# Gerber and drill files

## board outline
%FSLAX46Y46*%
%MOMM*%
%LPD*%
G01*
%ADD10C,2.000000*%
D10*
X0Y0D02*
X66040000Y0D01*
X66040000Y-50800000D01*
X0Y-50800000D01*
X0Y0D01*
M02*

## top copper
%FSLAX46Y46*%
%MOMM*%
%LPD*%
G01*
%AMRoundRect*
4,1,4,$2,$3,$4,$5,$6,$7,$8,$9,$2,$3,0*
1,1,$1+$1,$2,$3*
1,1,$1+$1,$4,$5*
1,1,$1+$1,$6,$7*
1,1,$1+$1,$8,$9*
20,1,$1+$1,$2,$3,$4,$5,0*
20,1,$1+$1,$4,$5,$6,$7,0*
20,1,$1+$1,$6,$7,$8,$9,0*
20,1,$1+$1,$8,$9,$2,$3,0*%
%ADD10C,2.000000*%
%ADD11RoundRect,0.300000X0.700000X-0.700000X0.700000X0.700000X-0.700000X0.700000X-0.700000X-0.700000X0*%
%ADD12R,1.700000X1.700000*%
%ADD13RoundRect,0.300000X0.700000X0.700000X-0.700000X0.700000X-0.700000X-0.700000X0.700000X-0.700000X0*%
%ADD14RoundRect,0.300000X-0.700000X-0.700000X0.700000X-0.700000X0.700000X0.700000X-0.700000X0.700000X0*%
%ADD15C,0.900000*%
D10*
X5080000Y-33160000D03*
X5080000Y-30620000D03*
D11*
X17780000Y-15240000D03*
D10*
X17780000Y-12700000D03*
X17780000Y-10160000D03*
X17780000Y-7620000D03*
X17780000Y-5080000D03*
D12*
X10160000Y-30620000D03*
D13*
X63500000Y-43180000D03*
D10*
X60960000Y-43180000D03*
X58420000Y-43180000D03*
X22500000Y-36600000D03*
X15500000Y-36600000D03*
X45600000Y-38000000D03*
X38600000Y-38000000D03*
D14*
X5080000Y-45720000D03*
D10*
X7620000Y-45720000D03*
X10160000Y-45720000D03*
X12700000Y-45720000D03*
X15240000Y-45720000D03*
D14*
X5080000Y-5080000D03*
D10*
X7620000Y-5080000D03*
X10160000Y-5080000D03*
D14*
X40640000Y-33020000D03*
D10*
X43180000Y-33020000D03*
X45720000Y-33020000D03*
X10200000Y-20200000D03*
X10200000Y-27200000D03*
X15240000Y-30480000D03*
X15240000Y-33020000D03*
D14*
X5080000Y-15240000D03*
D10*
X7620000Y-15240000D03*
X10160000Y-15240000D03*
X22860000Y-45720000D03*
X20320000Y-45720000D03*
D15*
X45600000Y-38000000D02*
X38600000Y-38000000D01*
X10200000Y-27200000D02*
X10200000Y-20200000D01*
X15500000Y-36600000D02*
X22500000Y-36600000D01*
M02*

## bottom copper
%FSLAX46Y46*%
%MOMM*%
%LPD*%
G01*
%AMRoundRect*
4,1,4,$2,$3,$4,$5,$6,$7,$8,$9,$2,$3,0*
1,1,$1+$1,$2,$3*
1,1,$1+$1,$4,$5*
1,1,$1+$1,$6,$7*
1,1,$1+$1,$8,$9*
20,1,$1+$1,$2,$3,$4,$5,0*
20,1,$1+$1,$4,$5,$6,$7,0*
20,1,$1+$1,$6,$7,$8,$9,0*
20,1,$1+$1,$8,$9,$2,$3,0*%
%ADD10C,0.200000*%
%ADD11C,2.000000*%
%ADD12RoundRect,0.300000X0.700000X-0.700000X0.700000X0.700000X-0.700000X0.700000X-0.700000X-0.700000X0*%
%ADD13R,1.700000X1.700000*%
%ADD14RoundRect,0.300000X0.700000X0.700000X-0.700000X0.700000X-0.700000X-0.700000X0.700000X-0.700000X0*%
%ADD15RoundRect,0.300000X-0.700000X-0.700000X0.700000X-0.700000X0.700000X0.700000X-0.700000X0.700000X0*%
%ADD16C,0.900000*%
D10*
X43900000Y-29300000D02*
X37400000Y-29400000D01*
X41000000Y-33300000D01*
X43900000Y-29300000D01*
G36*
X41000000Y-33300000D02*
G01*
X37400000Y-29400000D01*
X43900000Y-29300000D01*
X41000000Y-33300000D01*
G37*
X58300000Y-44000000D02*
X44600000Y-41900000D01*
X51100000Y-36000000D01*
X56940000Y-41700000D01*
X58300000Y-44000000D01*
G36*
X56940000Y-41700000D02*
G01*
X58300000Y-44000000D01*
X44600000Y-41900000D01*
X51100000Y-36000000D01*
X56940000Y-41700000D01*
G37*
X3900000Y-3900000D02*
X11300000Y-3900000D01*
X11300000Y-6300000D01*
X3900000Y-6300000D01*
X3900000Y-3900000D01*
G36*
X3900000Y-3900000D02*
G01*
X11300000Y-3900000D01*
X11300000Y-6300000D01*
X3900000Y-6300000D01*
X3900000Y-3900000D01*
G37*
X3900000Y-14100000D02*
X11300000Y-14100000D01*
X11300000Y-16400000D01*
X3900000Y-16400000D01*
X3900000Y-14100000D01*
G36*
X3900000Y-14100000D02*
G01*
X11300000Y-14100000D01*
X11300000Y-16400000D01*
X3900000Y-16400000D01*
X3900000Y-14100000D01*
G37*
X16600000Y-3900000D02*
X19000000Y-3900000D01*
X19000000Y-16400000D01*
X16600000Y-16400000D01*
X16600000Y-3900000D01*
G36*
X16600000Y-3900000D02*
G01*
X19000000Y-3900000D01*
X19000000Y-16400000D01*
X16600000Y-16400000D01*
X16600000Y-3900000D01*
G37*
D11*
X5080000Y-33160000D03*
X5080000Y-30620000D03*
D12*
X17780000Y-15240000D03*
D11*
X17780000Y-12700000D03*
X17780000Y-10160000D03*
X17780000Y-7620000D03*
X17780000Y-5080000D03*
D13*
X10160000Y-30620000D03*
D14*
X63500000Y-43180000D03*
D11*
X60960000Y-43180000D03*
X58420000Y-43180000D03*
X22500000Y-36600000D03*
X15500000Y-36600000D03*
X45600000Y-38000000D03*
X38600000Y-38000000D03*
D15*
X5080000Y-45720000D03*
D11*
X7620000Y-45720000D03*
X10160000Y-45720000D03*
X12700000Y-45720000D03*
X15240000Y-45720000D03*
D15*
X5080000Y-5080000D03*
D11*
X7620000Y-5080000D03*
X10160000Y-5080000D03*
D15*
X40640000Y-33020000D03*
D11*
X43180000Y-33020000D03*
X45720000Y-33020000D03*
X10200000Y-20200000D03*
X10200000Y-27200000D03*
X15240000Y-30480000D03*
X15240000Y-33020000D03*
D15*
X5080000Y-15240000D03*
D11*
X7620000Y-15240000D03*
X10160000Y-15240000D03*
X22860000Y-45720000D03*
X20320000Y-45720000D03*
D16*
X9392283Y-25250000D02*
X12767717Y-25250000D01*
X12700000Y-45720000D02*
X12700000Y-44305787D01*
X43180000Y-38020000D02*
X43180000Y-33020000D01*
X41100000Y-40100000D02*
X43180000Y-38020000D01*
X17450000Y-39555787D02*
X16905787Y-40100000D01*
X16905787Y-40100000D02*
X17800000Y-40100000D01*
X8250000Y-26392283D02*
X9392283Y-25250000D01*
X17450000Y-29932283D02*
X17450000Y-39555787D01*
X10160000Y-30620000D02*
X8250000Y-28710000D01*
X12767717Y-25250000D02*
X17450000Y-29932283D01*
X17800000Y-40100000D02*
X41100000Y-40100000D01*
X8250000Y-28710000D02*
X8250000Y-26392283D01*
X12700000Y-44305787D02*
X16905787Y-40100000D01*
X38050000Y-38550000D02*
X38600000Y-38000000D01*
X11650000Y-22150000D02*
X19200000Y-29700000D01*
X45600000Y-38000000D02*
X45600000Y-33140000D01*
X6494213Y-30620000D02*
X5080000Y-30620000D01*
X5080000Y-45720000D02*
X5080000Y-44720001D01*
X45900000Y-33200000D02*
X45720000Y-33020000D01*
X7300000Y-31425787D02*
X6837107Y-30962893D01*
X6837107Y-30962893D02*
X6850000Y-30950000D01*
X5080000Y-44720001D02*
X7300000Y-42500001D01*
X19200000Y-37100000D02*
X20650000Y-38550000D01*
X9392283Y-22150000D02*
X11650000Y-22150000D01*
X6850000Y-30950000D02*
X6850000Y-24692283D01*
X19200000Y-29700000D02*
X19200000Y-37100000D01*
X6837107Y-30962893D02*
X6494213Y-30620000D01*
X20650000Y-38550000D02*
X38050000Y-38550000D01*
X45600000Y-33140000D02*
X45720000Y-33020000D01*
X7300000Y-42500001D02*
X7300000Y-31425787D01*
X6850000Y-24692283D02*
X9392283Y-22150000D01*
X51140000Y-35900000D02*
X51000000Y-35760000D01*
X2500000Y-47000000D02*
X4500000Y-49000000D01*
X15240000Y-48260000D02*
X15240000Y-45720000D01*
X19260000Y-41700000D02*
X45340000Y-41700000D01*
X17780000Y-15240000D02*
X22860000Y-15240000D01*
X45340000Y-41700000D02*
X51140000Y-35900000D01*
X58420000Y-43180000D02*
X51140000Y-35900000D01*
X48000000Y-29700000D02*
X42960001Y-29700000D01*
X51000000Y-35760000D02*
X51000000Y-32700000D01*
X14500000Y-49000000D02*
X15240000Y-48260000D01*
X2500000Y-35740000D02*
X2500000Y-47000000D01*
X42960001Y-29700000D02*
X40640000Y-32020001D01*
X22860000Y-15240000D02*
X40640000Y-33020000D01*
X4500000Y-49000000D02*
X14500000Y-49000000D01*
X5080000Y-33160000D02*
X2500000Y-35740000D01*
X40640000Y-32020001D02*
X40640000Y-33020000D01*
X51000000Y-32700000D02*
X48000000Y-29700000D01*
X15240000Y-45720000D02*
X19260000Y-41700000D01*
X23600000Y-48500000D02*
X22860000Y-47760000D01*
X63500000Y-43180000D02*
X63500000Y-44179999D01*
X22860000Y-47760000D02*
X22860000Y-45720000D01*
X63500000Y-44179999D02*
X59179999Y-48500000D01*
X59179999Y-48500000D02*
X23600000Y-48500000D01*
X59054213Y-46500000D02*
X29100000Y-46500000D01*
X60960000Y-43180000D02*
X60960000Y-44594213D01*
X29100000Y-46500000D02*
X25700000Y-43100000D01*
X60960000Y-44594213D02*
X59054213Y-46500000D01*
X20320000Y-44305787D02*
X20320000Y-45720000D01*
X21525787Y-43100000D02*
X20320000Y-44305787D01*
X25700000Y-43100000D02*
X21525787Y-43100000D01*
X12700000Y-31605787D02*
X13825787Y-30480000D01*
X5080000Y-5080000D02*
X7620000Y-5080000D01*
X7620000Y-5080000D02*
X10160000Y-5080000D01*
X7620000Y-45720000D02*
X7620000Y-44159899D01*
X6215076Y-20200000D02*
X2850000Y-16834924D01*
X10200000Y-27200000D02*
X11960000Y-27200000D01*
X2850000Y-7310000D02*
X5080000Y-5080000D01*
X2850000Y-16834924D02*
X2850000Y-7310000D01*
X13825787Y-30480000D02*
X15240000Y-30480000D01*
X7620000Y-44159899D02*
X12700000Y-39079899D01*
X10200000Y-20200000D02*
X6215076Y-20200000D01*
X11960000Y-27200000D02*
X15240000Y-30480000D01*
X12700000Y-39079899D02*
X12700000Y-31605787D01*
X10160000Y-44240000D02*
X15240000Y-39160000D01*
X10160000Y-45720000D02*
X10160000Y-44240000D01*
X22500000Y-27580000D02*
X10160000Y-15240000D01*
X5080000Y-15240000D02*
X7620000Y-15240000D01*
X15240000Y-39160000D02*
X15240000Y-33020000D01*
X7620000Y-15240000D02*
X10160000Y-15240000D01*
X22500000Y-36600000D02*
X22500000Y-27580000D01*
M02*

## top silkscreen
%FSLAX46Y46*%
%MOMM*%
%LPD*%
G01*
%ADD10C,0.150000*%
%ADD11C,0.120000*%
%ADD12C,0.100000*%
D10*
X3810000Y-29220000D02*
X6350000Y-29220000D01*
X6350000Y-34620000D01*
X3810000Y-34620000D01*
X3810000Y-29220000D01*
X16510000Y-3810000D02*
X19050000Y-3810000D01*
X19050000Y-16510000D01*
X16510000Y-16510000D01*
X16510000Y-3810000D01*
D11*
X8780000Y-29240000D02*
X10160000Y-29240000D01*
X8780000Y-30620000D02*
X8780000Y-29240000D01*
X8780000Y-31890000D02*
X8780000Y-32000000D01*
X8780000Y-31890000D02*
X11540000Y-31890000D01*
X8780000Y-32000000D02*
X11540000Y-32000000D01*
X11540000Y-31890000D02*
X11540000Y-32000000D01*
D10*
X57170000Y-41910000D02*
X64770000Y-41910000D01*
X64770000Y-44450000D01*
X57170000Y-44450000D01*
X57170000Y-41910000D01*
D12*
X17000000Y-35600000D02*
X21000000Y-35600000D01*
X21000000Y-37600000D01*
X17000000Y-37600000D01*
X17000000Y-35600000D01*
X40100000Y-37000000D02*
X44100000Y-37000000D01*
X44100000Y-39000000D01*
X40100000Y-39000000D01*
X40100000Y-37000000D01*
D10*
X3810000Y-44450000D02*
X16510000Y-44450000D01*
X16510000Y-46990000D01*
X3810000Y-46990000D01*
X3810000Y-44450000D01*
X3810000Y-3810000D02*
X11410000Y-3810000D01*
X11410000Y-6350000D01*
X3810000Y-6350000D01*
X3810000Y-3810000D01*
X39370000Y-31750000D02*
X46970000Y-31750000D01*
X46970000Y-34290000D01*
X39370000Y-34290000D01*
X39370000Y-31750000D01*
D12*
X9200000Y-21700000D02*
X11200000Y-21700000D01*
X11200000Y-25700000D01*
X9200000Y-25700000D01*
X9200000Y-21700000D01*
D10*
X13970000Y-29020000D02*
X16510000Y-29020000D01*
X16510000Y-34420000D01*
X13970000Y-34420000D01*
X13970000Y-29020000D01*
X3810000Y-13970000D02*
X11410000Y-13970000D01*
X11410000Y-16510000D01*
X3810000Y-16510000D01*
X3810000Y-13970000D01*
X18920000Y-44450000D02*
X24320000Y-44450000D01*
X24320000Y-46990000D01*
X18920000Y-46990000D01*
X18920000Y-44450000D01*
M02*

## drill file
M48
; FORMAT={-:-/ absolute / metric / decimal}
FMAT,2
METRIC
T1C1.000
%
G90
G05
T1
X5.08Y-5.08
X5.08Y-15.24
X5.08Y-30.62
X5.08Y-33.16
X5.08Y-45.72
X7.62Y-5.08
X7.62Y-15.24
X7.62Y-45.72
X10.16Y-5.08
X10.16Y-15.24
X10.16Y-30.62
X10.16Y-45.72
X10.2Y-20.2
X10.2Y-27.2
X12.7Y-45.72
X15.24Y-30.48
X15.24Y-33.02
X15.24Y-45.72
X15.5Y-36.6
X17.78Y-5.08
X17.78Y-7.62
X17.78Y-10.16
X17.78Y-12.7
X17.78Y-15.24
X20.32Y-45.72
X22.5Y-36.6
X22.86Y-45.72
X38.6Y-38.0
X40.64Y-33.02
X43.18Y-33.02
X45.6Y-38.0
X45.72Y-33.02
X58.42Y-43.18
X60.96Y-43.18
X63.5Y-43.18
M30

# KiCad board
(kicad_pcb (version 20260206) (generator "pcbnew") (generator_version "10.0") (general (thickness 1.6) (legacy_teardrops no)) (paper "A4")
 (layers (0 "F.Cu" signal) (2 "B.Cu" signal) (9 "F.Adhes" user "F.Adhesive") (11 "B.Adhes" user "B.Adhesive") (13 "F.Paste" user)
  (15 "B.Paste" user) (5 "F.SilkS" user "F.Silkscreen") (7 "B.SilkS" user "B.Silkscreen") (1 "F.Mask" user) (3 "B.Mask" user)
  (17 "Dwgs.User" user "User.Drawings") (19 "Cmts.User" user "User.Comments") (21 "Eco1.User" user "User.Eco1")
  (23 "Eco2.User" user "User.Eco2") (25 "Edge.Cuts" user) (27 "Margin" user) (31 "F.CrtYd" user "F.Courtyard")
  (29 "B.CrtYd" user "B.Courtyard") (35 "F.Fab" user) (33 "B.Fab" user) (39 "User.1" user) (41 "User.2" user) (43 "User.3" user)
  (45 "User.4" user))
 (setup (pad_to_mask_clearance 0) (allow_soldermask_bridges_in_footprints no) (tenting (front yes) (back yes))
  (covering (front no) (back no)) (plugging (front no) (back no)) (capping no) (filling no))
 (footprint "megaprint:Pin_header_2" (layer "F.Cu") (at 5.08 31.82 90)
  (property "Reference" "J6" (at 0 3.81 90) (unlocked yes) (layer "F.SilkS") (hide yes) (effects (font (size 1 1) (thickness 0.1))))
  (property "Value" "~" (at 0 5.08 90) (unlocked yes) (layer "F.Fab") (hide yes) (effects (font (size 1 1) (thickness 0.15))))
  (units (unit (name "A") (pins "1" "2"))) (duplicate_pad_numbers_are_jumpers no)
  (fp_rect (start -2.8 -1.27) (end 2.6 1.27) (stroke (width 0.15) (type default)) (fill no) (layer "F.SilkS"))
  (pad "1" thru_hole circle (at -1.34 0 90) (size 2 2) (drill 1) (layers "*.Cu" "*.Mask") (remove_unused_layers no) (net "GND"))
  (pad "2" thru_hole circle (at 1.2 0 90) (size 2 2) (drill 1) (layers "*.Cu" "*.Mask") (remove_unused_layers no) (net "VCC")))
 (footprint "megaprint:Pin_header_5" (layer "F.Cu") (at 17.78 10.16 90)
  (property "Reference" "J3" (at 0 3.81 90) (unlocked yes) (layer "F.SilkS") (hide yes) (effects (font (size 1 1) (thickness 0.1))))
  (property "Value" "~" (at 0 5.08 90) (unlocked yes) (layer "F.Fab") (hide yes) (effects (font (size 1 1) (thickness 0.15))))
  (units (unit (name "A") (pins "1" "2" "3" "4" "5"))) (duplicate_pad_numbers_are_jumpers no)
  (fp_rect (start -6.35 -1.27) (end 6.35 1.27) (stroke (width 0.15) (type default)) (fill no) (layer "F.SilkS"))
  (pad "1" thru_hole roundrect (at -5.08 0 90) (size 2 2) (drill 1) (layers "*.Cu" "*.Mask") (remove_unused_layers no)
   (roundrect_rratio 0.15) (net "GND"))
  (pad "2" thru_hole circle (at -2.54 0 90) (size 2 2) (drill 1) (layers "*.Cu" "*.Mask") (remove_unused_layers no) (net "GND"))
  (pad "3" thru_hole circle (at 0 0 90) (size 2 2) (drill 1) (layers "*.Cu" "*.Mask") (remove_unused_layers no) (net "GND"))
  (pad "4" thru_hole circle (at 2.54 0 90) (size 2 2) (drill 1) (layers "*.Cu" "*.Mask") (remove_unused_layers no) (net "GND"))
  (pad "5" thru_hole circle (at 5.08 0 90) (size 2 2) (drill 1) (layers "*.Cu" "*.Mask") (remove_unused_layers no) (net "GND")))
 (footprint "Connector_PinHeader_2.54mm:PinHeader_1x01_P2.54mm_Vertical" (layer "F.Cu") (at 10.16 30.62)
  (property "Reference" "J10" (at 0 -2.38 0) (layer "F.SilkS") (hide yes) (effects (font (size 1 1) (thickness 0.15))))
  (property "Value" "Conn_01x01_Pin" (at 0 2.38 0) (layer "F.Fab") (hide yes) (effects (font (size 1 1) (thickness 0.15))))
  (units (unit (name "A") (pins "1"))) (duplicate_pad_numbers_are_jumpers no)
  (fp_line (start -1.38 -1.38) (end 0 -1.38) (stroke (width 0.12) (type solid)) (layer "F.SilkS"))
  (fp_line (start -1.38 0) (end -1.38 -1.38) (stroke (width 0.12) (type solid)) (layer "F.SilkS"))
  (fp_line (start -1.38 1.27) (end -1.38 1.38) (stroke (width 0.12) (type solid)) (layer "F.SilkS"))
  (fp_line (start -1.38 1.27) (end 1.38 1.27) (stroke (width 0.12) (type solid)) (layer "F.SilkS"))
  (fp_line (start -1.38 1.38) (end 1.38 1.38) (stroke (width 0.12) (type solid)) (layer "F.SilkS"))
  (fp_line (start 1.38 1.27) (end 1.38 1.38) (stroke (width 0.12) (type solid)) (layer "F.SilkS"))
  (pad "1" thru_hole rect (at 0 0) (size 1.7 1.7) (drill 1) (layers "*.Cu" "*.Mask") (remove_unused_layers no) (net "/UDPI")))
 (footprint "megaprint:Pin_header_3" (layer "F.Cu") (at 60.96 43.18 180)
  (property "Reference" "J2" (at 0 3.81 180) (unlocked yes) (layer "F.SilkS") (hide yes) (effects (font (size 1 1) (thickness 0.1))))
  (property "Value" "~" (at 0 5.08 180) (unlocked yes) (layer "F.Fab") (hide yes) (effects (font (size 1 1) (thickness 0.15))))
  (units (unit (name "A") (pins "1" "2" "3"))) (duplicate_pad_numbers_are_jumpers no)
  (fp_rect (start -3.81 -1.27) (end 3.79 1.27) (stroke (width 0.15) (type default)) (fill no) (layer "F.SilkS"))
  (pad "1" thru_hole roundrect (at -2.54 0 180) (size 2 2) (drill 1) (layers "*.Cu" "*.Mask") (remove_unused_layers no)
   (roundrect_rratio 0.15) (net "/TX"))
  (pad "2" thru_hole circle (at 0 0 180) (size 2 2) (drill 1) (layers "*.Cu" "*.Mask") (remove_unused_layers no) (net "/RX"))
  (pad "3" thru_hole circle (at 2.54 0 180) (size 2 2) (drill 1) (layers "*.Cu" "*.Mask") (remove_unused_layers no) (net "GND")))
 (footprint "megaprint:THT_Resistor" (layer "F.Cu") (at 19 36.6 180)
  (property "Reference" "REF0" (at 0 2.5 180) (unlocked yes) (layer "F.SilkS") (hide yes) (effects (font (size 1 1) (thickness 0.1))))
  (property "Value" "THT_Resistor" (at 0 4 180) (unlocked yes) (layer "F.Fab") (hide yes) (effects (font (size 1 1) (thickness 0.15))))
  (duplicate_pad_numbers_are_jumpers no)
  (fp_rect (start -2 -1) (end 2 1) (stroke (width 0.1) (type default)) (fill no) (layer "F.SilkS"))
  (pad "1" thru_hole circle (at -3.5 0 180) (size 2 2) (drill 1) (layers "*.Cu" "*.Mask") (remove_unused_layers no) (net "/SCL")
   (thermal_bridge_angle 90))
  (pad "2" thru_hole circle (at 3.5 0 180) (size 2 2) (drill 1) (layers "*.Cu" "*.Mask") (remove_unused_layers no) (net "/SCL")
   (thermal_bridge_angle 90)))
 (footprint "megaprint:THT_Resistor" (layer "F.Cu") (at 42.1 38 180)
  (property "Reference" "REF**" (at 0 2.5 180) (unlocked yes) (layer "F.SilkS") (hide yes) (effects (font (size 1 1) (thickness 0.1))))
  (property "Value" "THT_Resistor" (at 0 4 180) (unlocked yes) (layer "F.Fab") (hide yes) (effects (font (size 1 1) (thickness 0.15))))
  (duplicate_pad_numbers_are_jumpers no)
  (fp_rect (start -2 -1) (end 2 1) (stroke (width 0.1) (type default)) (fill no) (layer "F.SilkS"))
  (pad "1" thru_hole circle (at -3.5 0 180) (size 2 2) (drill 1) (layers "*.Cu" "*.Mask") (remove_unused_layers no) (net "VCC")
   (thermal_bridge_angle 90))
  (pad "2" thru_hole circle (at 3.5 0 180) (size 2 2) (drill 1) (layers "*.Cu" "*.Mask") (remove_unused_layers no) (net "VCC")
   (thermal_bridge_angle 90)))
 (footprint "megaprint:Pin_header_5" (layer "F.Cu") (at 10.16 45.72)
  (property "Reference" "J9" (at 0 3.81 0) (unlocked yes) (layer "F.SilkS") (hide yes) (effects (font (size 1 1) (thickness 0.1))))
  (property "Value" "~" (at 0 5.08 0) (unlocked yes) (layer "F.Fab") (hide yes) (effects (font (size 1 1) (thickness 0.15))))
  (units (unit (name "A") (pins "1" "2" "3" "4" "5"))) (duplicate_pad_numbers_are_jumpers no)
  (fp_rect (start -6.35 -1.27) (end 6.35 1.27) (stroke (width 0.15) (type default)) (fill no) (layer "F.SilkS"))
  (pad "1" thru_hole roundrect (at -5.08 0) (size 2 2) (drill 1) (layers "*.Cu" "*.Mask") (remove_unused_layers no) (roundrect_rratio 0.15)
   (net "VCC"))
  (pad "2" thru_hole circle (at -2.54 0) (size 2 2) (drill 1) (layers "*.Cu" "*.Mask") (remove_unused_layers no) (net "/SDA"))
  (pad "3" thru_hole circle (at 0 0) (size 2 2) (drill 1) (layers "*.Cu" "*.Mask") (remove_unused_layers no) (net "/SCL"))
  (pad "4" thru_hole circle (at 2.54 0) (size 2 2) (drill 1) (layers "*.Cu" "*.Mask") (remove_unused_layers no) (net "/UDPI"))
  (pad "5" thru_hole circle (at 5.08 0) (size 2 2) (drill 1) (layers "*.Cu" "*.Mask") (remove_unused_layers no) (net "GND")))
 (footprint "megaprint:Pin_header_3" (layer "F.Cu") (at 7.62 5.08)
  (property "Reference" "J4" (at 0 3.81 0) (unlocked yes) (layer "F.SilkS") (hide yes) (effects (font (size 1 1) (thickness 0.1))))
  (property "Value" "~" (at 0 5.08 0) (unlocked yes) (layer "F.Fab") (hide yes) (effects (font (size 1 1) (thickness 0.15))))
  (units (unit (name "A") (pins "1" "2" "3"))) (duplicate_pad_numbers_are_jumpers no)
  (fp_rect (start -3.81 -1.27) (end 3.79 1.27) (stroke (width 0.15) (type default)) (fill no) (layer "F.SilkS"))
  (pad "1" thru_hole roundrect (at -2.54 0) (size 2 2) (drill 1) (layers "*.Cu" "*.Mask") (remove_unused_layers no) (roundrect_rratio 0.15)
   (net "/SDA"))
  (pad "2" thru_hole circle (at 0 0) (size 2 2) (drill 1) (layers "*.Cu" "*.Mask") (remove_unused_layers no) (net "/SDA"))
  (pad "3" thru_hole circle (at 2.54 0) (size 2 2) (drill 1) (layers "*.Cu" "*.Mask") (remove_unused_layers no) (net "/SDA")))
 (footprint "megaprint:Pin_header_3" (layer "F.Cu") (at 43.18 33.02)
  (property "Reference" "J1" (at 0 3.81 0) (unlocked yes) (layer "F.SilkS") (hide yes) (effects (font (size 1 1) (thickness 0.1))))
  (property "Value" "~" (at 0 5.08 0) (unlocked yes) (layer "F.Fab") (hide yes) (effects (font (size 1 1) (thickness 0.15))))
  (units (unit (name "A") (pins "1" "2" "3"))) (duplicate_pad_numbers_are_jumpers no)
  (fp_rect (start -3.81 -1.27) (end 3.79 1.27) (stroke (width 0.15) (type default)) (fill no) (layer "F.SilkS"))
  (pad "1" thru_hole roundrect (at -2.54 0) (size 2 2) (drill 1) (layers "*.Cu" "*.Mask") (remove_unused_layers no) (roundrect_rratio 0.15)
   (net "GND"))
  (pad "2" thru_hole circle (at 0 0) (size 2 2) (drill 1) (layers "*.Cu" "*.Mask") (remove_unused_layers no) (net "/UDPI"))
  (pad "3" thru_hole circle (at 2.54 0) (size 2 2) (drill 1) (layers "*.Cu" "*.Mask") (remove_unused_layers no) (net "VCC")))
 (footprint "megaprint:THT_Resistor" (layer "F.Cu") (at 10.2 23.7 -90)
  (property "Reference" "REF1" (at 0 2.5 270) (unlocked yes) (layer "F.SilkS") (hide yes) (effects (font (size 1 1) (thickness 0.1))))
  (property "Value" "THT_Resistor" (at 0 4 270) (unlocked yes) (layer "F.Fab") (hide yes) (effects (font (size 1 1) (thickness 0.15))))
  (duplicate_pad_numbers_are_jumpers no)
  (fp_rect (start -2 -1) (end 2 1) (stroke (width 0.1) (type default)) (fill no) (layer "F.SilkS"))
  (pad "1" thru_hole circle (at -3.5 0 270) (size 2 2) (drill 1) (layers "*.Cu" "*.Mask") (remove_unused_layers no) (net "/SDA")
   (thermal_bridge_angle 90))
  (pad "2" thru_hole circle (at 3.5 0 270) (size 2 2) (drill 1) (layers "*.Cu" "*.Mask") (remove_unused_layers no) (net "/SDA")
   (thermal_bridge_angle 90)))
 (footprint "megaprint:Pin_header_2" (layer "F.Cu") (at 15.24 31.82 -90)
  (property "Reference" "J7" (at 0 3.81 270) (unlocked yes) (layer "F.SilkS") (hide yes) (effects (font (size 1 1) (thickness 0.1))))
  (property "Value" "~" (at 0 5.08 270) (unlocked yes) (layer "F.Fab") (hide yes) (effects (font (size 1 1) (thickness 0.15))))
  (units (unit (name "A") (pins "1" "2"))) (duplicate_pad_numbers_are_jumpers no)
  (fp_rect (start -2.8 -1.27) (end 2.6 1.27) (stroke (width 0.15) (type default)) (fill no) (layer "F.SilkS"))
  (pad "1" thru_hole circle (at -1.34 0 270) (size 2 2) (drill 1) (layers "*.Cu" "*.Mask") (remove_unused_layers no) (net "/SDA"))
  (pad "2" thru_hole circle (at 1.2 0 270) (size 2 2) (drill 1) (layers "*.Cu" "*.Mask") (remove_unused_layers no) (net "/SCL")))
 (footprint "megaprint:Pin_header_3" (layer "F.Cu") (at 7.62 15.24)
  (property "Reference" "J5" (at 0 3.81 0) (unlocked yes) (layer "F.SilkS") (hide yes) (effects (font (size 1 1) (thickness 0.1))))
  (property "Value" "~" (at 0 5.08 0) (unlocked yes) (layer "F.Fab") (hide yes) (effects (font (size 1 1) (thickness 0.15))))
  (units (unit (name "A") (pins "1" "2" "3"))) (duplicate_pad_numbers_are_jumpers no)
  (fp_rect (start -3.81 -1.27) (end 3.79 1.27) (stroke (width 0.15) (type default)) (fill no) (layer "F.SilkS"))
  (pad "1" thru_hole roundrect (at -2.54 0) (size 2 2) (drill 1) (layers "*.Cu" "*.Mask") (remove_unused_layers no) (roundrect_rratio 0.15)
   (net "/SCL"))
  (pad "2" thru_hole circle (at 0 0) (size 2 2) (drill 1) (layers "*.Cu" "*.Mask") (remove_unused_layers no) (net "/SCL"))
  (pad "3" thru_hole circle (at 2.54 0) (size 2 2) (drill 1) (layers "*.Cu" "*.Mask") (remove_unused_layers no) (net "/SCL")))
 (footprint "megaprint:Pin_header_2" (layer "F.Cu") (at 21.52 45.72 180)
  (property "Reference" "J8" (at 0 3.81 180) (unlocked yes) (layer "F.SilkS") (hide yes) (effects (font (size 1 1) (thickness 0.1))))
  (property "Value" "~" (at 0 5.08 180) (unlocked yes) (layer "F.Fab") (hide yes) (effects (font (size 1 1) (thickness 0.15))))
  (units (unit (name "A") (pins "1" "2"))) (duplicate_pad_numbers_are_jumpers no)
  (fp_rect (start -2.8 -1.27) (end 2.6 1.27) (stroke (width 0.15) (type default)) (fill no) (layer "F.SilkS"))
  (pad "1" thru_hole circle (at -1.34 0 180) (size 2 2) (drill 1) (layers "*.Cu" "*.Mask") (remove_unused_layers no) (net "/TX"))
  (pad "2" thru_hole circle (at 1.2 0 180) (size 2 2) (drill 1) (layers "*.Cu" "*.Mask") (remove_unused_layers no) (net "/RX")))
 (gr_poly (pts (xy 43.9 29.3) (xy 37.4 29.4) (xy 41 33.3)) (stroke (width 0.2) (type solid)) (fill yes) (layer "B.Cu") (net "GND"))
 (gr_poly
  (pts (xy 58.3 44) (xy 44.6 41.9) (xy 51.1 36) (xy 56.94 41.7)) (stroke (width 0.2) (type solid)) (fill yes) (layer "B.Cu") (net "GND"))
 (gr_rect (start 3.9 3.9) (end 11.3 6.3) (stroke (width 0.2) (type default)) (fill yes) (layer "B.Cu") (net "/SDA"))
 (gr_rect (start 3.9 14.1) (end 11.3 16.4) (stroke (width 0.2) (type default)) (fill yes) (layer "B.Cu") (net "/SCL"))
 (gr_rect (start 16.6 3.9) (end 19 16.4) (stroke (width 0.2) (type default)) (fill yes) (layer "B.Cu") (net "GND"))
 (gr_rect (start 0 0) (end 66.04 50.8) (stroke (width 2) (type solid)) (fill no) (layer "Edge.Cuts"))
 (segment (start 9.392283 25.25) (end 12.767717 25.25) (width 0.9) (layer "B.Cu") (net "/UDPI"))
 (segment (start 12.7 45.72) (end 12.7 44.305787) (width 0.9) (layer "B.Cu") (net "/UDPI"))
 (segment (start 43.18 38.02) (end 43.18 33.02) (width 0.9) (layer "B.Cu") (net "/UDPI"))
 (segment (start 41.1 40.1) (end 43.18 38.02) (width 0.9) (layer "B.Cu") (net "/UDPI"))
 (segment (start 17.45 39.555787) (end 16.905787 40.1) (width 0.9) (layer "B.Cu") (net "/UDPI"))
 (segment (start 16.905787 40.1) (end 17.8 40.1) (width 0.9) (layer "B.Cu") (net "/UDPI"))
 (segment (start 8.25 26.392283) (end 9.392283 25.25) (width 0.9) (layer "B.Cu") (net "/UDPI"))
 (segment (start 17.45 29.932283) (end 17.45 39.555787) (width 0.9) (layer "B.Cu") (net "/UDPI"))
 (segment (start 10.16 30.62) (end 8.25 28.71) (width 0.9) (layer "B.Cu") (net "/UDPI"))
 (segment (start 12.767717 25.25) (end 17.45 29.932283) (width 0.9) (layer "B.Cu") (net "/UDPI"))
 (segment (start 17.8 40.1) (end 41.1 40.1) (width 0.9) (layer "B.Cu") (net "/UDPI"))
 (segment (start 8.25 28.71) (end 8.25 26.392283) (width 0.9) (layer "B.Cu") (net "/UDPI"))
 (segment (start 12.7 44.305787) (end 16.905787 40.1) (width 0.9) (layer "B.Cu") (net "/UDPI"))
 (segment (start 45.6 38) (end 38.6 38) (width 0.9) (layer "F.Cu") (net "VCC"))
 (segment (start 38.05 38.55) (end 38.6 38) (width 0.9) (layer "B.Cu") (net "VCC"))
 (segment (start 11.65 22.15) (end 19.2 29.7) (width 0.9) (layer "B.Cu") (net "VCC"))
 (segment (start 45.6 38) (end 45.6 33.14) (width 0.9) (layer "B.Cu") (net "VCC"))
 (segment (start 6.494213 30.62) (end 5.08 30.62) (width 0.9) (layer "B.Cu") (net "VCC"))
 (segment (start 5.08 45.72) (end 5.08 44.720001) (width 0.9) (layer "B.Cu") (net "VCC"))
 (segment (start 45.9 33.2) (end 45.72 33.02) (width 0.9) (layer "B.Cu") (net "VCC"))
 (segment (start 7.3 31.425787) (end 6.837107 30.962893) (width 0.9) (layer "B.Cu") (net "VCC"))
 (segment (start 6.837107 30.962893) (end 6.85 30.95) (width 0.9) (layer "B.Cu") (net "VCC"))
 (segment (start 5.08 44.720001) (end 7.3 42.500001) (width 0.9) (layer "B.Cu") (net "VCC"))
 (segment (start 19.2 37.1) (end 20.65 38.55) (width 0.9) (layer "B.Cu") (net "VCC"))
 (segment (start 9.392283 22.15) (end 11.65 22.15) (width 0.9) (layer "B.Cu") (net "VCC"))
 (segment (start 6.85 30.95) (end 6.85 24.692283) (width 0.9) (layer "B.Cu") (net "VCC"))
 (segment (start 19.2 29.7) (end 19.2 37.1) (width 0.9) (layer "B.Cu") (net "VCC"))
 (segment (start 6.837107 30.962893) (end 6.494213 30.62) (width 0.9) (layer "B.Cu") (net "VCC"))
 (segment (start 20.65 38.55) (end 38.05 38.55) (width 0.9) (layer "B.Cu") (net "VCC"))
 (segment (start 45.6 33.14) (end 45.72 33.02) (width 0.9) (layer "B.Cu") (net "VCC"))
 (segment (start 7.3 42.500001) (end 7.3 31.425787) (width 0.9) (layer "B.Cu") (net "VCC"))
 (segment (start 6.85 24.692283) (end 9.392283 22.15) (width 0.9) (layer "B.Cu") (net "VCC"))
 (segment (start 51.14 35.9) (end 51 35.76) (width 0.9) (layer "B.Cu") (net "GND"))
 (segment (start 2.5 47) (end 4.5 49) (width 0.9) (layer "B.Cu") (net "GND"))
 (segment (start 15.24 48.26) (end 15.24 45.72) (width 0.9) (layer "B.Cu") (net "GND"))
 (segment (start 19.26 41.7) (end 45.34 41.7) (width 0.9) (layer "B.Cu") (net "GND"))
 (segment (start 17.78 15.24) (end 22.86 15.24) (width 0.9) (layer "B.Cu") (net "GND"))
 (segment (start 45.34 41.7) (end 51.14 35.9) (width 0.9) (layer "B.Cu") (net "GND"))
 (segment (start 58.42 43.18) (end 51.14 35.9) (width 0.9) (layer "B.Cu") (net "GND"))
 (segment (start 48 29.7) (end 42.960001 29.7) (width 0.9) (layer "B.Cu") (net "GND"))
 (segment (start 51 35.76) (end 51 32.7) (width 0.9) (layer "B.Cu") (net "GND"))
 (segment (start 14.5 49) (end 15.24 48.26) (width 0.9) (layer "B.Cu") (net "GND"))
 (segment (start 2.5 35.74) (end 2.5 47) (width 0.9) (layer "B.Cu") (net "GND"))
 (segment (start 42.960001 29.7) (end 40.64 32.020001) (width 0.9) (layer "B.Cu") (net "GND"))
 (segment (start 22.86 15.24) (end 40.64 33.02) (width 0.9) (layer "B.Cu") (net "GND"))
 (segment (start 4.5 49) (end 14.5 49) (width 0.9) (layer "B.Cu") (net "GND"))
 (segment (start 5.08 33.16) (end 2.5 35.74) (width 0.9) (layer "B.Cu") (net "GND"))
 (segment (start 40.64 32.020001) (end 40.64 33.02) (width 0.9) (layer "B.Cu") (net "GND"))
 (segment (start 51 32.7) (end 48 29.7) (width 0.9) (layer "B.Cu") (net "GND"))
 (segment (start 15.24 45.72) (end 19.26 41.7) (width 0.9) (layer "B.Cu") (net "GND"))
 (segment (start 23.6 48.5) (end 22.86 47.76) (width 0.9) (layer "B.Cu") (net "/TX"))
 (segment (start 63.5 43.18) (end 63.5 44.179999) (width 0.9) (layer "B.Cu") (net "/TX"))
 (segment (start 22.86 47.76) (end 22.86 45.72) (width 0.9) (layer "B.Cu") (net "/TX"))
 (segment (start 63.5 44.179999) (end 59.179999 48.5) (width 0.9) (layer "B.Cu") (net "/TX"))
 (segment (start 59.179999 48.5) (end 23.6 48.5) (width 0.9) (layer "B.Cu") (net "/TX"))
 (segment (start 59.054213 46.5) (end 29.1 46.5) (width 0.9) (layer "B.Cu") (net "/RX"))
 (segment (start 60.96 43.18) (end 60.96 44.594213) (width 0.9) (layer "B.Cu") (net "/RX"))
 (segment (start 29.1 46.5) (end 25.7 43.1) (width 0.9) (layer "B.Cu") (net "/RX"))
 (segment (start 60.96 44.594213) (end 59.054213 46.5) (width 0.9) (layer "B.Cu") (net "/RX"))
 (segment (start 20.32 44.305787) (end 20.32 45.72) (width 0.9) (layer "B.Cu") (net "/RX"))
 (segment (start 21.525787 43.1) (end 20.32 44.305787) (width 0.9) (layer "B.Cu") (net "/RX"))
 (segment (start 25.7 43.1) (end 21.525787 43.1) (width 0.9) (layer "B.Cu") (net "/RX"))
 (segment (start 10.2 27.2) (end 10.2 20.2) (width 0.9) (layer "F.Cu") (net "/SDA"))
 (segment (start 12.7 31.605787) (end 13.825787 30.48) (width 0.9) (layer "B.Cu") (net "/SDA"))
 (segment (start 5.08 5.08) (end 7.62 5.08) (width 0.9) (layer "B.Cu") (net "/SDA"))
 (segment (start 7.62 5.08) (end 10.16 5.08) (width 0.9) (layer "B.Cu") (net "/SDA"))
 (segment (start 7.62 45.72) (end 7.62 44.159899) (width 0.9) (layer "B.Cu") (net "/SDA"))
 (segment (start 6.215076 20.2) (end 2.85 16.834924) (width 0.9) (layer "B.Cu") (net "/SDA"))
 (segment (start 10.2 27.2) (end 11.96 27.2) (width 0.9) (layer "B.Cu") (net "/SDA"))
 (segment (start 2.85 7.31) (end 5.08 5.08) (width 0.9) (layer "B.Cu") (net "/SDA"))
 (segment (start 2.85 16.834924) (end 2.85 7.31) (width 0.9) (layer "B.Cu") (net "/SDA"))
 (segment (start 13.825787 30.48) (end 15.24 30.48) (width 0.9) (layer "B.Cu") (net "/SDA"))
 (segment (start 7.62 44.159899) (end 12.7 39.079899) (width 0.9) (layer "B.Cu") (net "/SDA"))
 (segment (start 10.2 20.2) (end 6.215076 20.2) (width 0.9) (layer "B.Cu") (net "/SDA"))
 (segment (start 11.96 27.2) (end 15.24 30.48) (width 0.9) (layer "B.Cu") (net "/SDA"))
 (segment (start 12.7 39.079899) (end 12.7 31.605787) (width 0.9) (layer "B.Cu") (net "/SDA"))
 (segment (start 15.5 36.6) (end 22.5 36.6) (width 0.9) (layer "F.Cu") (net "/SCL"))
 (segment (start 10.16 44.24) (end 15.24 39.16) (width 0.9) (layer "B.Cu") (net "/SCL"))
 (segment (start 10.16 45.72) (end 10.16 44.24) (width 0.9) (layer "B.Cu") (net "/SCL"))
 (segment (start 22.5 27.58) (end 10.16 15.24) (width 0.9) (layer "B.Cu") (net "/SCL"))
 (segment (start 5.08 15.24) (end 7.62 15.24) (width 0.9) (layer "B.Cu") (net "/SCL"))
 (segment (start 15.24 39.16) (end 15.24 33.02) (width 0.9) (layer "B.Cu") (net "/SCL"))
 (segment (start 7.62 15.24) (end 10.16 15.24) (width 0.9) (layer "B.Cu") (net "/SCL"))
 (segment (start 22.5 36.6) (end 22.5 27.58) (width 0.9) (layer "B.Cu") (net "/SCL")))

